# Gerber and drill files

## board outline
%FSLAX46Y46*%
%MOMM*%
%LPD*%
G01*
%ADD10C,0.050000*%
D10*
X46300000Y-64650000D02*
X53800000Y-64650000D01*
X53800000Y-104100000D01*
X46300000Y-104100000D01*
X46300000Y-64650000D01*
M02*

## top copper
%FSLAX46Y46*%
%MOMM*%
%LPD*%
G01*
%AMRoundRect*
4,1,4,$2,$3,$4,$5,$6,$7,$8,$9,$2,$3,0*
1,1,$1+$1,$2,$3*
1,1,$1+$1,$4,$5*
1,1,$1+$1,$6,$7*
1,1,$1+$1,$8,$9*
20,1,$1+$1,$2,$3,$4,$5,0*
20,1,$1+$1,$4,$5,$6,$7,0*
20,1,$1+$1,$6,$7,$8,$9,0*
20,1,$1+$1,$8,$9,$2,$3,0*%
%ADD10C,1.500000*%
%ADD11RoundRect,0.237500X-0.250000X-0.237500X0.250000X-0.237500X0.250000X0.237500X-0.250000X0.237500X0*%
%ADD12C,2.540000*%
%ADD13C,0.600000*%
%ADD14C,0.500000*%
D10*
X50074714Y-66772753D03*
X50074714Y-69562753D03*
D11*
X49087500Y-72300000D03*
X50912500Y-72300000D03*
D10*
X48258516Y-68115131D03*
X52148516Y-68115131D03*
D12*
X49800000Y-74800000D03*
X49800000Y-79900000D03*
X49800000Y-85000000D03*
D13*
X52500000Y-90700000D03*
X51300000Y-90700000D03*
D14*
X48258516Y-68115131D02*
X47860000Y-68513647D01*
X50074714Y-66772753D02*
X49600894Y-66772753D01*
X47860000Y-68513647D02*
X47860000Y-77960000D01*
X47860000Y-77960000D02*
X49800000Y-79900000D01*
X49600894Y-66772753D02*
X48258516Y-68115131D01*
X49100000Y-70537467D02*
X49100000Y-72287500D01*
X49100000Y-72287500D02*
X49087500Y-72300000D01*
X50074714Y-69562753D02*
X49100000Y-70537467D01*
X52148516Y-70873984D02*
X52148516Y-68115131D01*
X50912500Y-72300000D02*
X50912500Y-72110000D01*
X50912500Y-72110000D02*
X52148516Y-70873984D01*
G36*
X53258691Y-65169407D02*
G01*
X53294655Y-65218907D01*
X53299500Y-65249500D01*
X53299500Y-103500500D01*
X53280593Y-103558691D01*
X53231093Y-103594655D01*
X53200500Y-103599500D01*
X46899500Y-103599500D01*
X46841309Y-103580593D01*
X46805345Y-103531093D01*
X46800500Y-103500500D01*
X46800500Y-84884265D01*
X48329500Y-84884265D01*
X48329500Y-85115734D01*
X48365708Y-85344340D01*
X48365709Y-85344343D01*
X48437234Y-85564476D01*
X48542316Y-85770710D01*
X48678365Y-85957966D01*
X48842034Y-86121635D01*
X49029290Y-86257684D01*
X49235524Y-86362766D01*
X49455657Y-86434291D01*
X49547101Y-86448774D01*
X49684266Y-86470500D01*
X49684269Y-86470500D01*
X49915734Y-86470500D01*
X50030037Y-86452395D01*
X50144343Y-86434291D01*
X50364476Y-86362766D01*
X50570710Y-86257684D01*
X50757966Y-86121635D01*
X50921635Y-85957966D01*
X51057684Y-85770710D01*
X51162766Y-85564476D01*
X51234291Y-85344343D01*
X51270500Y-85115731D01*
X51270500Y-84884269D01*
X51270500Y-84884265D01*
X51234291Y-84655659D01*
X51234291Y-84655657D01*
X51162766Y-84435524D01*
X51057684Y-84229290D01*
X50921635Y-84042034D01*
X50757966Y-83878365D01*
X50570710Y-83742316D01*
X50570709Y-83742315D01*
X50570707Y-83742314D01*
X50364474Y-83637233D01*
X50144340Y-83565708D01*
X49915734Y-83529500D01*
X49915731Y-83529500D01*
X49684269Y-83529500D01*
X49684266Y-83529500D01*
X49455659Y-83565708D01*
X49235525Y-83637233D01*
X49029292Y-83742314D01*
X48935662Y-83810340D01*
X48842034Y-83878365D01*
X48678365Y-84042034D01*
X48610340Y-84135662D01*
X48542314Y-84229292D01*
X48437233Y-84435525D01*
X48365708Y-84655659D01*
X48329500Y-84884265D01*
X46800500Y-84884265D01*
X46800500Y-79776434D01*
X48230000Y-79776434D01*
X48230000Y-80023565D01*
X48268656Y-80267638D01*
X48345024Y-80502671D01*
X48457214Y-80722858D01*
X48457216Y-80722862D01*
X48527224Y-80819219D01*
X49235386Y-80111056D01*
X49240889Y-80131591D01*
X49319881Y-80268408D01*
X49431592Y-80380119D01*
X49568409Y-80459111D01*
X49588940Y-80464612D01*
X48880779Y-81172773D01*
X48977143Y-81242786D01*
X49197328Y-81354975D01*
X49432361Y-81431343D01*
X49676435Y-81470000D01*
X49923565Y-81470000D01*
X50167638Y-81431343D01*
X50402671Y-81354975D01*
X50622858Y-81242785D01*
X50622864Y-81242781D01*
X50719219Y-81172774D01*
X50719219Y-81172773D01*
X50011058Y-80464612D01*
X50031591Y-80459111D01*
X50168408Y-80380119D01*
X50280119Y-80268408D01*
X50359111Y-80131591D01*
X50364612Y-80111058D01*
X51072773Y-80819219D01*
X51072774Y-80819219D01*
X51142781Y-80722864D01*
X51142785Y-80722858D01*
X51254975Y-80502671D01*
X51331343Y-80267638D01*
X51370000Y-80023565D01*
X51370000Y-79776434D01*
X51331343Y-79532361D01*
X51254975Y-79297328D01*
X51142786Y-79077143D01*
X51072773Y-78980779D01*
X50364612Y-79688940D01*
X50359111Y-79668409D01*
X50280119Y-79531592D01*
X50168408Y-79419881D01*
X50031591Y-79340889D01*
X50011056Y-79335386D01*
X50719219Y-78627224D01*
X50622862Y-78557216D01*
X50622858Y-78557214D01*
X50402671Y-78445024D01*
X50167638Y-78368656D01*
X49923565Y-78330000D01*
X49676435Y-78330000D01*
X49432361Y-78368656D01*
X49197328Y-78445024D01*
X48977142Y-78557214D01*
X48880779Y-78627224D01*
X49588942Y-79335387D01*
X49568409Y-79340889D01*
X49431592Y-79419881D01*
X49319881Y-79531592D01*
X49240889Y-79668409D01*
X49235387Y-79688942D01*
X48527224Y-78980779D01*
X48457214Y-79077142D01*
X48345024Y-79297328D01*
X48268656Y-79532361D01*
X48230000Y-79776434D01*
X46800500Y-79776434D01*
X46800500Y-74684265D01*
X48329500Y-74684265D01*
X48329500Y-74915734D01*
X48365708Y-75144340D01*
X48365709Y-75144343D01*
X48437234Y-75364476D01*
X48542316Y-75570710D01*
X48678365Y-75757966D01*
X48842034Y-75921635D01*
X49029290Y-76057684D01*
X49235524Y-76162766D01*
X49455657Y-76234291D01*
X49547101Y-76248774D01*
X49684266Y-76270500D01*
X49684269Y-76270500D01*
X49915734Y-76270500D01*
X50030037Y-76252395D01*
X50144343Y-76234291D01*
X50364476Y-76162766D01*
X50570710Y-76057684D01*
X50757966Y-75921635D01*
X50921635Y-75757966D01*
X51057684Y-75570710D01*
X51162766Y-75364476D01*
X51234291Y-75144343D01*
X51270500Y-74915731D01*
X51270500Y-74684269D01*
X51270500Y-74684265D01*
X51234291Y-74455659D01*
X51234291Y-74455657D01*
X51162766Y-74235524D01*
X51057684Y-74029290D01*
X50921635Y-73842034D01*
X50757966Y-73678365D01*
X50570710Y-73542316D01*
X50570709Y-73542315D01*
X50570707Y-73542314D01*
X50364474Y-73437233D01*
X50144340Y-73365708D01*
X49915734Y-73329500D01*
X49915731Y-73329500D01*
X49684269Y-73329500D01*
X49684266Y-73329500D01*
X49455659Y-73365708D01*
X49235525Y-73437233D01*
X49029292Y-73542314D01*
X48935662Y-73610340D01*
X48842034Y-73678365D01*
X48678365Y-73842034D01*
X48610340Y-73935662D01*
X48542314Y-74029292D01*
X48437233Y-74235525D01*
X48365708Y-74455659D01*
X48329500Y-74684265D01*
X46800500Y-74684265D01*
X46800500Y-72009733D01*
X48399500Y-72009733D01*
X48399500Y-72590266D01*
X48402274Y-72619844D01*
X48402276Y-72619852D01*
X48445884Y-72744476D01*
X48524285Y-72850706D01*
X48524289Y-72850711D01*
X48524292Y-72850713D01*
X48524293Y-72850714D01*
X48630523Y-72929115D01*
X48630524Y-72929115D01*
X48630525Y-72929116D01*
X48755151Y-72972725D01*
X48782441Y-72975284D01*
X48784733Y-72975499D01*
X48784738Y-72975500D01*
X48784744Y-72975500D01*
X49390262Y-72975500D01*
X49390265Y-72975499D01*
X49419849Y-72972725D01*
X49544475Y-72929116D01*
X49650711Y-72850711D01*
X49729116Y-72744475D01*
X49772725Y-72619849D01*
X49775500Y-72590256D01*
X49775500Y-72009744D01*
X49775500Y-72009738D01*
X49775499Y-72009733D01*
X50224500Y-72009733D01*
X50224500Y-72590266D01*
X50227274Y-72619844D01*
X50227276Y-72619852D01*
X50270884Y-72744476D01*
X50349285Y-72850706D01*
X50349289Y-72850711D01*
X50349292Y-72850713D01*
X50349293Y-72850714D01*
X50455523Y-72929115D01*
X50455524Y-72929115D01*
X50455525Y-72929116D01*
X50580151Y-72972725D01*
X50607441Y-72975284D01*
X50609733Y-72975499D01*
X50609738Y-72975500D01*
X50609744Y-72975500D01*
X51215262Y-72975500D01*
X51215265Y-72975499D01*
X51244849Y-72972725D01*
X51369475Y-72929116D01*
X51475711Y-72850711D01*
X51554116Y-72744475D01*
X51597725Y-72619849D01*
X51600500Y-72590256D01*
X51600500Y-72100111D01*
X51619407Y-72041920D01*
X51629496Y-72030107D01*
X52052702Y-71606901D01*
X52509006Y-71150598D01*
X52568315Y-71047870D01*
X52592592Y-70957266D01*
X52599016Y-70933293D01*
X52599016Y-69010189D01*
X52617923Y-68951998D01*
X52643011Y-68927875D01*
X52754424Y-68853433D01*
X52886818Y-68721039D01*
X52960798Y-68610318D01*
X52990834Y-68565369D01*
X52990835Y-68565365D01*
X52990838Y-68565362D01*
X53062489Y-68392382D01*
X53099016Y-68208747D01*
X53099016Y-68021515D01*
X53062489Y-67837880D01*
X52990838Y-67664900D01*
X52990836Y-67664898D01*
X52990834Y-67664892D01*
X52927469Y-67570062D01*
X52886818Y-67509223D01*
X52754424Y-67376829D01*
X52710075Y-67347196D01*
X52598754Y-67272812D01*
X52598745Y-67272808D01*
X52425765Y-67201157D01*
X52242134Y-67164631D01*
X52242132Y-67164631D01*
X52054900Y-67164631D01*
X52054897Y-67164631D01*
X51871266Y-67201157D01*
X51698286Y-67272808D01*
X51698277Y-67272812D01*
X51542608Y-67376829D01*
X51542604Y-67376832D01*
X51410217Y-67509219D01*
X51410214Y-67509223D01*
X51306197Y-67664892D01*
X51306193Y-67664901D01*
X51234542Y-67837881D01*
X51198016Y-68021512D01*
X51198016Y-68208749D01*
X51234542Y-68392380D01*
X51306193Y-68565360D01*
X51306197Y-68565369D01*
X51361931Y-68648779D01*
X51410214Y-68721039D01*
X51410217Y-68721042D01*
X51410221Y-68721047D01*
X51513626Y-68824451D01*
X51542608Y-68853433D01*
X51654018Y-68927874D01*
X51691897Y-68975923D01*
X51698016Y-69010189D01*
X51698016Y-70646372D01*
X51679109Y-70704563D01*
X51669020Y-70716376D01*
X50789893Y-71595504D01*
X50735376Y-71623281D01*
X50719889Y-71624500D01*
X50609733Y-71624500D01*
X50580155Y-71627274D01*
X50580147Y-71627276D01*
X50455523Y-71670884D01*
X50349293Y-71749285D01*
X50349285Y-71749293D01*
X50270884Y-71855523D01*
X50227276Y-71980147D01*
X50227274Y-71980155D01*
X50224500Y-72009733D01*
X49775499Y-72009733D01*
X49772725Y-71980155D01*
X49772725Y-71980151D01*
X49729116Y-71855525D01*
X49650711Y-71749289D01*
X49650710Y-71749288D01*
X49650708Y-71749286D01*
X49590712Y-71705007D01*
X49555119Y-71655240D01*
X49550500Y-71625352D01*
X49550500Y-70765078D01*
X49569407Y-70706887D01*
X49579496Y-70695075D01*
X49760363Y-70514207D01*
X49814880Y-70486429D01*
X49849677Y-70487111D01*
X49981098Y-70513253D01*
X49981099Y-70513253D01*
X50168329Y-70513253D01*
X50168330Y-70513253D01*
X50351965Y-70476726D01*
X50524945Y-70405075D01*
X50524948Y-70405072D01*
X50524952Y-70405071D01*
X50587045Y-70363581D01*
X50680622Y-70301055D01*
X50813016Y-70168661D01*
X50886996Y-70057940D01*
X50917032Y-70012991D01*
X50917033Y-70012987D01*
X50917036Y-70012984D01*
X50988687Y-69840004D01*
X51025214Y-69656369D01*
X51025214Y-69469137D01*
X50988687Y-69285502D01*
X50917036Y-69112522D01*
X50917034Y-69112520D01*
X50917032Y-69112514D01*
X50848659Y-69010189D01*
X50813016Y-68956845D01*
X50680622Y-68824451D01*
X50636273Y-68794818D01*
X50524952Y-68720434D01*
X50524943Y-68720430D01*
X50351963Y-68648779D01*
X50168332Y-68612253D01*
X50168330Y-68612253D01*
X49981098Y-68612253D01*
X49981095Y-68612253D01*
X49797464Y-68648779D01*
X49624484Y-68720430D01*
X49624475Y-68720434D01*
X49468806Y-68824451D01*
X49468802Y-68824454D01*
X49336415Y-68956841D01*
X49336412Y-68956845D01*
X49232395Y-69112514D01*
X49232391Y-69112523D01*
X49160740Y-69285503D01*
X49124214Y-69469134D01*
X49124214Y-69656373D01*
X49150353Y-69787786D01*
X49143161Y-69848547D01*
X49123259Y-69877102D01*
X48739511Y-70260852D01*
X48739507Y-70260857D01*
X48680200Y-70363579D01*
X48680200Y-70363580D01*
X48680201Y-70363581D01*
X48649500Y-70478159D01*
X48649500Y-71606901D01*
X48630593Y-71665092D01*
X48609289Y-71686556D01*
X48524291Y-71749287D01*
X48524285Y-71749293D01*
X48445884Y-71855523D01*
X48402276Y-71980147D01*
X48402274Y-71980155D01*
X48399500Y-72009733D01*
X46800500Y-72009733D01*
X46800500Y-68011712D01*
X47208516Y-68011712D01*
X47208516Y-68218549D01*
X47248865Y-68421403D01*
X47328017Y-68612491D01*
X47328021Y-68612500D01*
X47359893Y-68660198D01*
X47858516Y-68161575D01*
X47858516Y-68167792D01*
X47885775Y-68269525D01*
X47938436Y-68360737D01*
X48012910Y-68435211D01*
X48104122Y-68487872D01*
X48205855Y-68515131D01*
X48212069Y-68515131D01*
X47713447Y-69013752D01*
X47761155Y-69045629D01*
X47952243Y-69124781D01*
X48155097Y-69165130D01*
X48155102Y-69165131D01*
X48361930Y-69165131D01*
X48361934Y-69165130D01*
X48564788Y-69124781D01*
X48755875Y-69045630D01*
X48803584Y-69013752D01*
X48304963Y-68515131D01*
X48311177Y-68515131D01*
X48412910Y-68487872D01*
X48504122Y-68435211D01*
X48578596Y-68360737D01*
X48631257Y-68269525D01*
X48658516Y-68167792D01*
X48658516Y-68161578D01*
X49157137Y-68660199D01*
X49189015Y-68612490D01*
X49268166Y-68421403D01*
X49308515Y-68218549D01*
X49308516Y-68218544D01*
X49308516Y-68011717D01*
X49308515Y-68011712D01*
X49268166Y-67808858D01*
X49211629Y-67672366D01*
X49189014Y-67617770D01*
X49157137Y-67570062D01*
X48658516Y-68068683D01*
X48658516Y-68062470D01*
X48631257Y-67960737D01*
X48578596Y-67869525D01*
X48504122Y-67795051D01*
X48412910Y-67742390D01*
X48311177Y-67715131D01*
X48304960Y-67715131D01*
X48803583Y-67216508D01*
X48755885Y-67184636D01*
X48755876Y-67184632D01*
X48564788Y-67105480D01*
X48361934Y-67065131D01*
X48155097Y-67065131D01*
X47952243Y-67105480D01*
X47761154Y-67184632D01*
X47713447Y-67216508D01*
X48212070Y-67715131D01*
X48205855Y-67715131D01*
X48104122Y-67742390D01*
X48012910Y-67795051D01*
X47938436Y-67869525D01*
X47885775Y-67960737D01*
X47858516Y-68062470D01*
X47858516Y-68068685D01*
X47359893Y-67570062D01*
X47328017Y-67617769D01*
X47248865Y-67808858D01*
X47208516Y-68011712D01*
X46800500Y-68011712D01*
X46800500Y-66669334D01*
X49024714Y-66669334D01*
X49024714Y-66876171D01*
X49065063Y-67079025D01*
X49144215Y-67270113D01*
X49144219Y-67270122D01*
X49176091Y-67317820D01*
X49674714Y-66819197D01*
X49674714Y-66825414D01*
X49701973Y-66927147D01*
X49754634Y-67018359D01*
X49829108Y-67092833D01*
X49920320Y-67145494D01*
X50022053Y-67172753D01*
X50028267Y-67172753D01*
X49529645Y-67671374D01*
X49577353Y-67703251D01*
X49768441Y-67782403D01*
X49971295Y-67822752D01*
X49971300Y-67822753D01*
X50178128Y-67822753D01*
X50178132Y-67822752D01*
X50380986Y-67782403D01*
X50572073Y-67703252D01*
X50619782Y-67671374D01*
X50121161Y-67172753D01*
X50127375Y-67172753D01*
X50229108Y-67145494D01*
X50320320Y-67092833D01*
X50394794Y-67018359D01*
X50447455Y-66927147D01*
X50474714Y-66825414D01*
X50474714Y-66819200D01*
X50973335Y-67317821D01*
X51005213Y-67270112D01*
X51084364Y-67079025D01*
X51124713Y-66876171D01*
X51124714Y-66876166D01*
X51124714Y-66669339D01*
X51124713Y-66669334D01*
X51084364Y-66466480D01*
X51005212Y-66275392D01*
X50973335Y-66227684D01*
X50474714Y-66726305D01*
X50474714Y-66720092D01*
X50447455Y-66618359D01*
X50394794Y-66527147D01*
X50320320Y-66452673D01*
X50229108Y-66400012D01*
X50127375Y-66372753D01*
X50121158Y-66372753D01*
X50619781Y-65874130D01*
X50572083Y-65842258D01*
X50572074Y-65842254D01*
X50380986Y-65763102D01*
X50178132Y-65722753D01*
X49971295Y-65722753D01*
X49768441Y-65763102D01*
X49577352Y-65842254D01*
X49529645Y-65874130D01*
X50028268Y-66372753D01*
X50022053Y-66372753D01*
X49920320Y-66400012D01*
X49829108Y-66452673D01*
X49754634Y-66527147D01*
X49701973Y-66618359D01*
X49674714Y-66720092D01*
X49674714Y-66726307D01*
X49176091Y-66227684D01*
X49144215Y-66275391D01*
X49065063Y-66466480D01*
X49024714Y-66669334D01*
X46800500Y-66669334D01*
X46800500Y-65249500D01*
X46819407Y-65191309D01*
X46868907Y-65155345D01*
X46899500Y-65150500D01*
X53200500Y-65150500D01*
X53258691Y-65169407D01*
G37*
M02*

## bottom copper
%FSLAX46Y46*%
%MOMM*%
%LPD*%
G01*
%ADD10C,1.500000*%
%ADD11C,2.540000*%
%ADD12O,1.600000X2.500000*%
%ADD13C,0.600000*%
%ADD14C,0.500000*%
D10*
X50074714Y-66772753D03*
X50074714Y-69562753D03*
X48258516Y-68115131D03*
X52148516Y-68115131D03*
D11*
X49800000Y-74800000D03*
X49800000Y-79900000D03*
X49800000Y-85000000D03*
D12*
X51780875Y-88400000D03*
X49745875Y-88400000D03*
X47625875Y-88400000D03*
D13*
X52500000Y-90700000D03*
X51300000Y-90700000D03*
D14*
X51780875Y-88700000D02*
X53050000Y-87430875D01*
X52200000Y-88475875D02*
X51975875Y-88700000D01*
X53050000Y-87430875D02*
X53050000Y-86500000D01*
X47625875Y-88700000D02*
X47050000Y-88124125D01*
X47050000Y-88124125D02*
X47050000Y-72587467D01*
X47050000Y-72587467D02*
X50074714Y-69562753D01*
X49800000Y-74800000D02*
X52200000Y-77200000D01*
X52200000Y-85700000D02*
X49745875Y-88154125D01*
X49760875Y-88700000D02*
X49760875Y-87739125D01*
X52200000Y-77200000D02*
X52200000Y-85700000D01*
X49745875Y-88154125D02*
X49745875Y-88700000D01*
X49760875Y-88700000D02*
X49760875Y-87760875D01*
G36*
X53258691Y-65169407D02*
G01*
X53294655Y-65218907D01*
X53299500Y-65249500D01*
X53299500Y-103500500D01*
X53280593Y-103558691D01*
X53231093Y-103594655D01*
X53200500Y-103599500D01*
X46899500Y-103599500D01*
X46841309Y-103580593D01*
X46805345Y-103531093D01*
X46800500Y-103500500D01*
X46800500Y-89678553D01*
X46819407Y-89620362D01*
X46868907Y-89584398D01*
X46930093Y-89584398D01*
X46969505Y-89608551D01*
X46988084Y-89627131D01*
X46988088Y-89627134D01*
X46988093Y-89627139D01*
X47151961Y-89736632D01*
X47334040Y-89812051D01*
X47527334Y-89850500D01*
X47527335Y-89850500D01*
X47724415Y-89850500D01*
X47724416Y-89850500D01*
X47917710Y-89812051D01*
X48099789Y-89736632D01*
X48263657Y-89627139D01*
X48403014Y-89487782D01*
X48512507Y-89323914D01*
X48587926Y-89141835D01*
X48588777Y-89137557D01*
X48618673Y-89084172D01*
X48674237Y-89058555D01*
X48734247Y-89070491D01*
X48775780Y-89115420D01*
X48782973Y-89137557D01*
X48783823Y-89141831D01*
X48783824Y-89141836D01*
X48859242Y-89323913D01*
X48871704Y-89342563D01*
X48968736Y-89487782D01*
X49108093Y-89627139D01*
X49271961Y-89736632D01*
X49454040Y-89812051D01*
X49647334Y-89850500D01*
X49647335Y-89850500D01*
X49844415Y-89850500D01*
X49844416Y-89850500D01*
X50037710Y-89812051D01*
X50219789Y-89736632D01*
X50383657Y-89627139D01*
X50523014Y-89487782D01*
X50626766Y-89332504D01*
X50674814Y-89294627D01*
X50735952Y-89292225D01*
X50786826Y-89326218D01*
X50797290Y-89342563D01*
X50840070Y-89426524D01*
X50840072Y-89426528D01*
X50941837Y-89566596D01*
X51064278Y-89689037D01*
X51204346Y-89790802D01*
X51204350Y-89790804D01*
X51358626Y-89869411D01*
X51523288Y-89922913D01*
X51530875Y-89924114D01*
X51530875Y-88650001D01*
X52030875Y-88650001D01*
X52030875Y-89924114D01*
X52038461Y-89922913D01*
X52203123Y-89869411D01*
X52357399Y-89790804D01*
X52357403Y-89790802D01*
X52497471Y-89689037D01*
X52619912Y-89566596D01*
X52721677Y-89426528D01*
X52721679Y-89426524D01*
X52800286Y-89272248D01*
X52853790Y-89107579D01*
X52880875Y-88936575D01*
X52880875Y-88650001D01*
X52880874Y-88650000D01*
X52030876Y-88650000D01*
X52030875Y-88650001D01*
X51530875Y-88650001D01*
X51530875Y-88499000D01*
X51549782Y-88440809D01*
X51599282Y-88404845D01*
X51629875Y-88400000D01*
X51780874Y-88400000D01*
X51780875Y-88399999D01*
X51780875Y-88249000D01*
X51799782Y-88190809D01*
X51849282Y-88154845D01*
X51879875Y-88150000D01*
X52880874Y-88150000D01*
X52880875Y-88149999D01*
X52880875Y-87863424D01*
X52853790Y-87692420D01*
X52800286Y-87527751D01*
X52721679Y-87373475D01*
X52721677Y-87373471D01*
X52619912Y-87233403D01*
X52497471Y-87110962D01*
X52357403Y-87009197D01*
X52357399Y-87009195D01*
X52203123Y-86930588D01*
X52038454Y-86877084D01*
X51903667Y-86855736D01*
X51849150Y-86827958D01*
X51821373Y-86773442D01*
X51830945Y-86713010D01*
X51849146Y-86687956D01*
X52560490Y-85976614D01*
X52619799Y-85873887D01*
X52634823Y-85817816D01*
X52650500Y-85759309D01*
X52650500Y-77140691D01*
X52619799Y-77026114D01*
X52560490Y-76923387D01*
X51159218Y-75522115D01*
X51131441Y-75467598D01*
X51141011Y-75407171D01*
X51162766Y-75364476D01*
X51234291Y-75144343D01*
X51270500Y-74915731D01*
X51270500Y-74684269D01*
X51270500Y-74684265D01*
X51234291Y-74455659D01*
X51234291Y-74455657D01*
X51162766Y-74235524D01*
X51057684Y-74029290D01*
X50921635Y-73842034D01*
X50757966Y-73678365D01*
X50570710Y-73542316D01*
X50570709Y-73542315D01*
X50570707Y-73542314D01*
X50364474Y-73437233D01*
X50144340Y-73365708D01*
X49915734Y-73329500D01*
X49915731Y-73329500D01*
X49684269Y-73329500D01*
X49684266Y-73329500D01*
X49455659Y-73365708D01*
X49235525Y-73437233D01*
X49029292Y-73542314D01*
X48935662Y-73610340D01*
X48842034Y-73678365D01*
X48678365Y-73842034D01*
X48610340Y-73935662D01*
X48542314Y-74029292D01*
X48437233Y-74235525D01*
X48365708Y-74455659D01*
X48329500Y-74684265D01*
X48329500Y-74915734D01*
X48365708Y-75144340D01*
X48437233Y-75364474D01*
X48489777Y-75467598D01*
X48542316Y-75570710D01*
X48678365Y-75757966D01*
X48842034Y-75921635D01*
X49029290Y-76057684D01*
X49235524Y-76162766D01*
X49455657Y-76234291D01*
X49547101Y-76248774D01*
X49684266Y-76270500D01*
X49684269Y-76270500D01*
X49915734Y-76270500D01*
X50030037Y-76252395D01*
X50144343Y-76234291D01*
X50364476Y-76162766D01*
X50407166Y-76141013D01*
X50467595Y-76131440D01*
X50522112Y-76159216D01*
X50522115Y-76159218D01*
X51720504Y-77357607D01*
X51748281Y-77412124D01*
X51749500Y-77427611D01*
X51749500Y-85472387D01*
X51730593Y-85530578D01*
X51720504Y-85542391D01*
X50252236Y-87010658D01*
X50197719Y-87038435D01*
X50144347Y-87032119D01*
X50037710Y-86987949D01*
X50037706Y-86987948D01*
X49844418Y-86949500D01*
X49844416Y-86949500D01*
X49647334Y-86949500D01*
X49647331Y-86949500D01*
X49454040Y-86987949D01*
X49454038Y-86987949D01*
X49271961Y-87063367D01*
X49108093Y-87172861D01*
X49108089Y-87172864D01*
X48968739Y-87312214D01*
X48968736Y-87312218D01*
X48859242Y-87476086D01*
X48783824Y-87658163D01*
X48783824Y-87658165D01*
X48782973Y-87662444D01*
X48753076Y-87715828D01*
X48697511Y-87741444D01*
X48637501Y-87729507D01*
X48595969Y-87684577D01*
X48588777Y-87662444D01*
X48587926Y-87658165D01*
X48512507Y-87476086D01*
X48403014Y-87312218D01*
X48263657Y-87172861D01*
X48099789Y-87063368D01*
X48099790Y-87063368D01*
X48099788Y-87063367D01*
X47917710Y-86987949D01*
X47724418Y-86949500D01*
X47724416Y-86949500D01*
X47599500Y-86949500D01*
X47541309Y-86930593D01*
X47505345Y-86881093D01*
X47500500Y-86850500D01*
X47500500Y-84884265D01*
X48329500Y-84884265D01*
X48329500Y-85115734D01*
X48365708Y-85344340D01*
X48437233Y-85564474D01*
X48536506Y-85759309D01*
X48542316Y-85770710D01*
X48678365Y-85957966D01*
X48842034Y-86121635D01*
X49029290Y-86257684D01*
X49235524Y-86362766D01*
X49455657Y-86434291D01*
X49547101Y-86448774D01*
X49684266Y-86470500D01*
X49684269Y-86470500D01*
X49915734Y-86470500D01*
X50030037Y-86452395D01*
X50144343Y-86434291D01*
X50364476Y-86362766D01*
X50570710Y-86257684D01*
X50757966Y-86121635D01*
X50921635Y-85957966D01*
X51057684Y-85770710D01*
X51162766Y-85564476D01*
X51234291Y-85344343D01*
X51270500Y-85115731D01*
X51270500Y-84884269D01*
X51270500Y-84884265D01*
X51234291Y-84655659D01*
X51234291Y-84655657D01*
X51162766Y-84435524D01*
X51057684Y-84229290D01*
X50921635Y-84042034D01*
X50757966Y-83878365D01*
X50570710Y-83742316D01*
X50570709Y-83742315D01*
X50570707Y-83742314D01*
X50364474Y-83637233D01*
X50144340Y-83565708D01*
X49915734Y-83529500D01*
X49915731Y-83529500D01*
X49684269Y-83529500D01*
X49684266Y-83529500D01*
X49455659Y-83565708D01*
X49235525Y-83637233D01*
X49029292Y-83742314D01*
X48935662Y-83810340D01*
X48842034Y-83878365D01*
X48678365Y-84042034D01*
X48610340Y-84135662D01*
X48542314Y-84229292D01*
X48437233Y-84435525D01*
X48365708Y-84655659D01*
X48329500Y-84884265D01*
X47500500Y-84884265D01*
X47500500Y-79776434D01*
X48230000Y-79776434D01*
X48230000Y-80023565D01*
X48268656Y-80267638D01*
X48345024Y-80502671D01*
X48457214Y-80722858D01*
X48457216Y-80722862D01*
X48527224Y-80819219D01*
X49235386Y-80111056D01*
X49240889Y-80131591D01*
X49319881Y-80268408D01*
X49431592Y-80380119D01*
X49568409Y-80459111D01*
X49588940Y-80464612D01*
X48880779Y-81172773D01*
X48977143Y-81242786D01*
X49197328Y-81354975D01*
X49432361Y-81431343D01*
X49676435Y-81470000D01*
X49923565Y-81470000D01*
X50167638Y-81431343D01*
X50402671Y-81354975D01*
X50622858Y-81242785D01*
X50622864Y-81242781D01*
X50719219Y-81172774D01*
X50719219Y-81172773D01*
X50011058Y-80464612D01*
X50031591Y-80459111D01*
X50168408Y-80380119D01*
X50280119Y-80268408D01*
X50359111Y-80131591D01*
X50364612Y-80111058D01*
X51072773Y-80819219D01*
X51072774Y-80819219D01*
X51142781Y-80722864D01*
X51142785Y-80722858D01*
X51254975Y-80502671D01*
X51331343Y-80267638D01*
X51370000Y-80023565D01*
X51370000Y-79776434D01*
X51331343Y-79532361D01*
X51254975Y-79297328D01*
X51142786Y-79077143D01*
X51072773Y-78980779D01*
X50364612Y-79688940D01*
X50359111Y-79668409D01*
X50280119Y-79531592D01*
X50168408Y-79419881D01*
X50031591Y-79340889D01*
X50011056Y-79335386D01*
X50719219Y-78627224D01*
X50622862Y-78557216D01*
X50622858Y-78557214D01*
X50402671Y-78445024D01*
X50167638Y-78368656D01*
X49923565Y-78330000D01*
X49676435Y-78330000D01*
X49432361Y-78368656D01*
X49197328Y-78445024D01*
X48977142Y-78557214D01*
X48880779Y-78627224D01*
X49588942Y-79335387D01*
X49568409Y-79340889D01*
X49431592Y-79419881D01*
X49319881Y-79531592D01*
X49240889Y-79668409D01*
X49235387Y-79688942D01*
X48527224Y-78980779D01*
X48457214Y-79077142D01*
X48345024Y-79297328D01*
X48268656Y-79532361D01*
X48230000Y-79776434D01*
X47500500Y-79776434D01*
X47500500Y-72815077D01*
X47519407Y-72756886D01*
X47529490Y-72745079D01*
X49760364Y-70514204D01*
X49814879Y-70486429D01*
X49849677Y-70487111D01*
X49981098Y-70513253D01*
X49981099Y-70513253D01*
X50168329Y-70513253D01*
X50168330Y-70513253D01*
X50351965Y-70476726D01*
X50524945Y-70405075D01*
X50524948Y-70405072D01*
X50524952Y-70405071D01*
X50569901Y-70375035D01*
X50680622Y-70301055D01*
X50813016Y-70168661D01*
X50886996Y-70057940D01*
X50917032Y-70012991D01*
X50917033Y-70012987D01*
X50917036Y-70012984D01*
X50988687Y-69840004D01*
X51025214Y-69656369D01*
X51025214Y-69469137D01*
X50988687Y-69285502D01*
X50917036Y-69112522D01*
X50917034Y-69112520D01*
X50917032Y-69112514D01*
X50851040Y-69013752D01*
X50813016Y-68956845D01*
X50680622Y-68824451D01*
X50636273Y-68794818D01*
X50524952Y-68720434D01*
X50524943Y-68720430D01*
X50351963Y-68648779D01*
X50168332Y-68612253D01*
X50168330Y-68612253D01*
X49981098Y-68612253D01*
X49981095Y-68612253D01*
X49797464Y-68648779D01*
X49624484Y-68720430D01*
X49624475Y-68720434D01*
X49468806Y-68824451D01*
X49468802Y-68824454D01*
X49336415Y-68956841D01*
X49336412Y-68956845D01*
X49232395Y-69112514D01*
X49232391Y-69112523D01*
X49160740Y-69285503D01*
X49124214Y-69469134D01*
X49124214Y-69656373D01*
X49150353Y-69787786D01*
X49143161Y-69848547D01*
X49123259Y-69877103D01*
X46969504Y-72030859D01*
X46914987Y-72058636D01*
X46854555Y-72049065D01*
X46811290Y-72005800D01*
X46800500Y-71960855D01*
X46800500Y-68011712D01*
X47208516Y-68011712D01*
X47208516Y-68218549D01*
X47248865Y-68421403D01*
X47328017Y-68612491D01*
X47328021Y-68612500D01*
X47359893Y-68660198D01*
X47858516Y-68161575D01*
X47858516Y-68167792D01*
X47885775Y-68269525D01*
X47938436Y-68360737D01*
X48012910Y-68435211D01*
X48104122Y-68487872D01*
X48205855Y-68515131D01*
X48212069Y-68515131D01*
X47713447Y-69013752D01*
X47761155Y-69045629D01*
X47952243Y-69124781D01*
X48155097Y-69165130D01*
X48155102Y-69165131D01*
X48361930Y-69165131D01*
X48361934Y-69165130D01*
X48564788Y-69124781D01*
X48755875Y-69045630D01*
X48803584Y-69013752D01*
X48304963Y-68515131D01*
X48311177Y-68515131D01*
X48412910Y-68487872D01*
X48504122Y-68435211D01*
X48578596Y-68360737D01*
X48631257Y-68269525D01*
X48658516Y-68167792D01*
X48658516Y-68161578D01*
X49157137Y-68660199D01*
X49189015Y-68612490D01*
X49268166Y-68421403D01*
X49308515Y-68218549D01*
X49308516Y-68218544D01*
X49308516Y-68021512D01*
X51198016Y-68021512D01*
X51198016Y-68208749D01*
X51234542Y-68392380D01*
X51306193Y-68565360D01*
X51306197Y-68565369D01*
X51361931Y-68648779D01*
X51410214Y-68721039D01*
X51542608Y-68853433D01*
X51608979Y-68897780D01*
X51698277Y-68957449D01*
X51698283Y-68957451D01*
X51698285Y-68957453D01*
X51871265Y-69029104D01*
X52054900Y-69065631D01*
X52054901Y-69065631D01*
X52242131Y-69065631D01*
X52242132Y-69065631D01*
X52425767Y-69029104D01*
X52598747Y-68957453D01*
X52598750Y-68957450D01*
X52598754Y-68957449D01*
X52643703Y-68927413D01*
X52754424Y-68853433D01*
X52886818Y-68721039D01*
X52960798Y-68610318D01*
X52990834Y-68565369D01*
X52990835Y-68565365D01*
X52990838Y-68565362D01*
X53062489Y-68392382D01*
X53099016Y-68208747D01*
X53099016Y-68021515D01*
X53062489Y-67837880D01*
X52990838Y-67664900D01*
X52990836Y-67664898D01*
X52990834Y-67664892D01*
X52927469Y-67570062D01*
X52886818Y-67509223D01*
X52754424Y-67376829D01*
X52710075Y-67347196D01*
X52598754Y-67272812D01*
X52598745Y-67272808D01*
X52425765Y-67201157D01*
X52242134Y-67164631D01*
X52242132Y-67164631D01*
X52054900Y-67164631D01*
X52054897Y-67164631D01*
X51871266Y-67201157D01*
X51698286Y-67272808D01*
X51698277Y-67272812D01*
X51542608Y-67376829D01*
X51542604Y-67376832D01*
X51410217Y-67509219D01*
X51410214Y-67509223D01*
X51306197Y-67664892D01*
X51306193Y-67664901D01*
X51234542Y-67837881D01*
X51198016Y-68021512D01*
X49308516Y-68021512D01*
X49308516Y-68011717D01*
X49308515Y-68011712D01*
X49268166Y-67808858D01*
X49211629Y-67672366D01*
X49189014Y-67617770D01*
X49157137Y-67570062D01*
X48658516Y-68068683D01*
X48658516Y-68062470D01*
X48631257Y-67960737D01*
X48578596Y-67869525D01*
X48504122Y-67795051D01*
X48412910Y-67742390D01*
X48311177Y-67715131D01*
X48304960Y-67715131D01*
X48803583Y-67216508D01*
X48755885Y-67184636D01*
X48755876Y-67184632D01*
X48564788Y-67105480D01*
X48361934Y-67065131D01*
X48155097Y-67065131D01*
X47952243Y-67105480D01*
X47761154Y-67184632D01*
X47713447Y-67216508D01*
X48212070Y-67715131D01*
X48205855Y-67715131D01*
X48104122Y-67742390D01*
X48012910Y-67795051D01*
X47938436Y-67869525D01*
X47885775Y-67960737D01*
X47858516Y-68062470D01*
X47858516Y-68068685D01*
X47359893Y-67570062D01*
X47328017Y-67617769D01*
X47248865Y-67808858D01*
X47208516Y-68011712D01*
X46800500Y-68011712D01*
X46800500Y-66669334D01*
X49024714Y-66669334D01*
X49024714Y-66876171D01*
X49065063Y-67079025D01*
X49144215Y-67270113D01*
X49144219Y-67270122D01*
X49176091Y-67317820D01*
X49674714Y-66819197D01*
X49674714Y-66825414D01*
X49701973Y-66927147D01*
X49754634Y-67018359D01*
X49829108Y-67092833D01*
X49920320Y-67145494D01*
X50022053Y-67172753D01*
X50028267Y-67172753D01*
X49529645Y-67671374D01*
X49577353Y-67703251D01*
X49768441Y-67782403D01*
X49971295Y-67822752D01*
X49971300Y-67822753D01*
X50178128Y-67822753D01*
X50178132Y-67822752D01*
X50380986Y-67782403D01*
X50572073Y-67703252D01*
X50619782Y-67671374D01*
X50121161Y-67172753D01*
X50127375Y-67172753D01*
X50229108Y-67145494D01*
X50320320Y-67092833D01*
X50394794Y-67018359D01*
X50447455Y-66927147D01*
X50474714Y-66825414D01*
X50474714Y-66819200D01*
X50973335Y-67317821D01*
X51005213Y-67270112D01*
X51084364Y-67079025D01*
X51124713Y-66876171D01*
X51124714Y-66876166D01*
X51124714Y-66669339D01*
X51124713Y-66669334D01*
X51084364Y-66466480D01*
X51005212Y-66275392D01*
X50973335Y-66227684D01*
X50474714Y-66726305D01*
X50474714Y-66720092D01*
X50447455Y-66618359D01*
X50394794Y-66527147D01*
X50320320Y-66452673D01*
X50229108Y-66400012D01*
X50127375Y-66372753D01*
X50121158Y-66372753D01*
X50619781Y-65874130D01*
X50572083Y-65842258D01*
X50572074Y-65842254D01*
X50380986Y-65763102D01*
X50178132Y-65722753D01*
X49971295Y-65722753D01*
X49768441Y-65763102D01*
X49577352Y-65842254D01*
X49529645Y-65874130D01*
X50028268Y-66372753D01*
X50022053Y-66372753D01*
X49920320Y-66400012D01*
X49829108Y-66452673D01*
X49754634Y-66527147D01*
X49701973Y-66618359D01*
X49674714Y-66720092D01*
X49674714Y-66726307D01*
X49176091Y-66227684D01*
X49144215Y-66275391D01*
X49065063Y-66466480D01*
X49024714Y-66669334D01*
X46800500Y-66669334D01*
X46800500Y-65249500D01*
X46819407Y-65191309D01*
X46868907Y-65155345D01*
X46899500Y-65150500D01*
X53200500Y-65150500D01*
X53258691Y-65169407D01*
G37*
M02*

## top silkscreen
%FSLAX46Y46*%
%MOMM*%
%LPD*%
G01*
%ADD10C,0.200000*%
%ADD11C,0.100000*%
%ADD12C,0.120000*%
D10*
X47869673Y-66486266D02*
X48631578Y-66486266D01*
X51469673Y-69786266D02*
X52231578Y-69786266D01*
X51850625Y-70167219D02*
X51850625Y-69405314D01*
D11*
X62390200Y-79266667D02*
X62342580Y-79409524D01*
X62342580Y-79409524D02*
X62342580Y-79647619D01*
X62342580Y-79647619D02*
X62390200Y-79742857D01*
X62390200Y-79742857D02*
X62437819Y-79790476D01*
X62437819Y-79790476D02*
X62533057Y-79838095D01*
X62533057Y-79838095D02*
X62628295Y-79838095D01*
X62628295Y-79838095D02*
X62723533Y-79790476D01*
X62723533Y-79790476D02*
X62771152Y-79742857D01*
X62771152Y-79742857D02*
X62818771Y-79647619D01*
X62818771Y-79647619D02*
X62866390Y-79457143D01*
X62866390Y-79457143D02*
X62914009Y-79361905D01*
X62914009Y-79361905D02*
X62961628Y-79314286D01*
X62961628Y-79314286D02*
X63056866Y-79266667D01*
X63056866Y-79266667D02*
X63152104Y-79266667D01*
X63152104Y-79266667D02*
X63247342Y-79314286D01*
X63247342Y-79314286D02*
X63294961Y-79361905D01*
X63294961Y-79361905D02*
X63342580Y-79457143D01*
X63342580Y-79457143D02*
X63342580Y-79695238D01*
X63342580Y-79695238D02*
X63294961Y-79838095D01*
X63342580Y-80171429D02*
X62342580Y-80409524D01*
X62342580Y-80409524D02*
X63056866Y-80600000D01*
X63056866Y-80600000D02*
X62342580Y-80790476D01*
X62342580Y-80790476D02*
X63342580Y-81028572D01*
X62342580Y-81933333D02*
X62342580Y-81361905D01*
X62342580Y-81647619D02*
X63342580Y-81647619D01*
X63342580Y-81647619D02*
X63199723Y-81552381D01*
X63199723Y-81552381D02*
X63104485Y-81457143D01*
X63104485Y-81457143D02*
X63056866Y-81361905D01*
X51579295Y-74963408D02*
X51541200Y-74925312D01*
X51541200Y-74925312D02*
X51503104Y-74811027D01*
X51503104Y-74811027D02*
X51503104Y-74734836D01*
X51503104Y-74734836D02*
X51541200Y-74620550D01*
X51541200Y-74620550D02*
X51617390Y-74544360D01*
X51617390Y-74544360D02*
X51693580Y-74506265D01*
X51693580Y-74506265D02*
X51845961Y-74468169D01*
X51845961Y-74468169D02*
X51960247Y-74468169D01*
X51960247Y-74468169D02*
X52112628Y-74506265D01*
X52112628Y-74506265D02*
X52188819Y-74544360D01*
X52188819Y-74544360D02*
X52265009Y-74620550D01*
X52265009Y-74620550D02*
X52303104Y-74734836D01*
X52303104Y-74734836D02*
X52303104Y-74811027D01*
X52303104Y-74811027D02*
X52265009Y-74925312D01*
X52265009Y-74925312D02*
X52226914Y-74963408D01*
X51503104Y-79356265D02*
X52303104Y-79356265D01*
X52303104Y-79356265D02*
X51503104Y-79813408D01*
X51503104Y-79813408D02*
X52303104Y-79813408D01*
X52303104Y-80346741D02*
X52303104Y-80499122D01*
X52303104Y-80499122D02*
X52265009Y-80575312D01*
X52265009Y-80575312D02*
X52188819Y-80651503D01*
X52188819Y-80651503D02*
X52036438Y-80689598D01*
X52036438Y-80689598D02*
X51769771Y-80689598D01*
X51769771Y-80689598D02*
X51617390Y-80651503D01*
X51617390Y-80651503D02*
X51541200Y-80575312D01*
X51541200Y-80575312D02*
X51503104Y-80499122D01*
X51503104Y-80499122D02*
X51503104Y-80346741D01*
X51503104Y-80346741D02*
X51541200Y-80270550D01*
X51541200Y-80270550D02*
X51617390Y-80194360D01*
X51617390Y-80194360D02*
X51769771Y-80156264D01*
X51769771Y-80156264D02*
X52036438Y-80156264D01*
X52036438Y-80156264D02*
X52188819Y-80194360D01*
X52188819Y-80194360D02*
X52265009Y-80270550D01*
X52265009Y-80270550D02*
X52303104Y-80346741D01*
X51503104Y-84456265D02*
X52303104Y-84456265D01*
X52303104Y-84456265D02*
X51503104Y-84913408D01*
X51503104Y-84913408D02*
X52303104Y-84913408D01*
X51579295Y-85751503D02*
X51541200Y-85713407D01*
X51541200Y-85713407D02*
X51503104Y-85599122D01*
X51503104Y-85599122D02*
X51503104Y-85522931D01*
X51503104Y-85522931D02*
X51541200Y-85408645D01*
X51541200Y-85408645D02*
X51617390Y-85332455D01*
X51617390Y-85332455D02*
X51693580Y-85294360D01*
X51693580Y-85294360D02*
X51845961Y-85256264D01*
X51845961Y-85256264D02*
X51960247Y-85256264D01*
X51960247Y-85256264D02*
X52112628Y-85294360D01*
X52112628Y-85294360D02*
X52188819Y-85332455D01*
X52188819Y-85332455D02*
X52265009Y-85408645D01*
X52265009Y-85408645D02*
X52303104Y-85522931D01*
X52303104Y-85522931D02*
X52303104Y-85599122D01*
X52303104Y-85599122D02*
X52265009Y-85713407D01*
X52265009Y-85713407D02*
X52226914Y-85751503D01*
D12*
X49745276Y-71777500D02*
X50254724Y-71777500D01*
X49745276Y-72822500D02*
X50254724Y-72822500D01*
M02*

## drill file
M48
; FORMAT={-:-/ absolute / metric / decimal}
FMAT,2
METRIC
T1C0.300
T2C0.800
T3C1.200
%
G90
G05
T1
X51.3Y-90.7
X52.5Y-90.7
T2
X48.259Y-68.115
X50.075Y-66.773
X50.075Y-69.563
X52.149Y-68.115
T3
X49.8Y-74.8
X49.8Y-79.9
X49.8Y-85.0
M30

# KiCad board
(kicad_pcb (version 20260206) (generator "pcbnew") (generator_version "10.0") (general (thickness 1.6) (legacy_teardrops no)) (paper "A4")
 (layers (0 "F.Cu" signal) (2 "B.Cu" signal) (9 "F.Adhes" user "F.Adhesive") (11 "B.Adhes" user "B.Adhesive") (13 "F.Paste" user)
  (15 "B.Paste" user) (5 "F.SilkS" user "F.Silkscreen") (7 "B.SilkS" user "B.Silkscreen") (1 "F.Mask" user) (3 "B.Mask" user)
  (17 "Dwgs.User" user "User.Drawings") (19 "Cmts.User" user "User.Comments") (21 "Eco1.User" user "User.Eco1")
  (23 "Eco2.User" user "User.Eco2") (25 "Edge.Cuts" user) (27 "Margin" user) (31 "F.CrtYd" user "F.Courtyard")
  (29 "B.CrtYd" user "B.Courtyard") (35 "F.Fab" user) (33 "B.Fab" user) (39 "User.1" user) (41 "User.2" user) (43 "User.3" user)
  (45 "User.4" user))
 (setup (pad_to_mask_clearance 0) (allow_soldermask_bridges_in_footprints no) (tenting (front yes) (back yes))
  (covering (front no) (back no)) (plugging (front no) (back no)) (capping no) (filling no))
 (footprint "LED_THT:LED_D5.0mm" (layer "F.Cu") (at 50.074714 66.872753 -90)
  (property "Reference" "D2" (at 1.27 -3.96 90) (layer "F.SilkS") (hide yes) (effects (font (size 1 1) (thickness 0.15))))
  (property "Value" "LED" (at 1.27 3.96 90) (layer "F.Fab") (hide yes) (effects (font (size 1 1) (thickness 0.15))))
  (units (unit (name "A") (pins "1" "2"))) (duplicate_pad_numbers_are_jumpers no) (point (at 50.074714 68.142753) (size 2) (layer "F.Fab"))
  (pad "1" thru_hole circle (at -0.1 0 270) (size 1.5 1.5) (drill 0.8) (layers "*.Cu" "*.Mask") (remove_unused_layers no) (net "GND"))
  (pad "2" thru_hole circle (at 2.69 0 270) (size 1.5 1.5) (drill 0.8) (layers "*.Cu" "*.Mask") (remove_unused_layers no) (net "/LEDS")))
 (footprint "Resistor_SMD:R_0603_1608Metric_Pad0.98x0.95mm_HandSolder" (layer "F.Cu") (at 50 72.3)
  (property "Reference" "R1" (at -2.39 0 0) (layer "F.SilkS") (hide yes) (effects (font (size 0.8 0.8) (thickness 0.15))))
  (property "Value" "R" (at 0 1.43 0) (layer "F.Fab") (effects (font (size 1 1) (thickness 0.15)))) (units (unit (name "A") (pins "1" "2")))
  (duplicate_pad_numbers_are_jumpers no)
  (fp_line (start -0.254724 -0.5225) (end 0.254724 -0.5225) (stroke (width 0.12) (type solid)) (layer "F.SilkS"))
  (fp_line (start -0.254724 0.5225) (end 0.254724 0.5225) (stroke (width 0.12) (type solid)) (layer "F.SilkS"))
  (pad "1" smd roundrect (at -0.9125 0) (size 0.975 0.95) (layers "F.Cu" "F.Mask" "F.Paste") (roundrect_rratio 0.25) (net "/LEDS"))
  (pad "2" smd roundrect (at 0.9125 0) (size 0.975 0.95) (layers "F.Cu" "F.Mask" "F.Paste") (roundrect_rratio 0.25) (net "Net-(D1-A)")))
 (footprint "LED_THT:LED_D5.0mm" (layer "F.Cu") (at 48.708516 68.115131)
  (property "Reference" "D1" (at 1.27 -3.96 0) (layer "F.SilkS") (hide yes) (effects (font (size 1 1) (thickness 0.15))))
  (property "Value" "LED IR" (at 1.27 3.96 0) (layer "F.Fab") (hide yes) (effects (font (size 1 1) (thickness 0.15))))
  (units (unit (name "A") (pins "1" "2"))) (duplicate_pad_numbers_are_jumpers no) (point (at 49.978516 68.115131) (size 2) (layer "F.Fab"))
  (pad "1" thru_hole circle (at -0.45 0) (size 1.5 1.5) (drill 0.8) (layers "*.Cu" "*.Mask") (remove_unused_layers no) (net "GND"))
  (pad "2" thru_hole circle (at 3.44 0) (size 1.5 1.5) (drill 0.8) (layers "*.Cu" "*.Mask") (remove_unused_layers no) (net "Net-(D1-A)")))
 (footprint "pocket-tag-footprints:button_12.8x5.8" (layer "F.Cu") (at 49.8 80.6 -90)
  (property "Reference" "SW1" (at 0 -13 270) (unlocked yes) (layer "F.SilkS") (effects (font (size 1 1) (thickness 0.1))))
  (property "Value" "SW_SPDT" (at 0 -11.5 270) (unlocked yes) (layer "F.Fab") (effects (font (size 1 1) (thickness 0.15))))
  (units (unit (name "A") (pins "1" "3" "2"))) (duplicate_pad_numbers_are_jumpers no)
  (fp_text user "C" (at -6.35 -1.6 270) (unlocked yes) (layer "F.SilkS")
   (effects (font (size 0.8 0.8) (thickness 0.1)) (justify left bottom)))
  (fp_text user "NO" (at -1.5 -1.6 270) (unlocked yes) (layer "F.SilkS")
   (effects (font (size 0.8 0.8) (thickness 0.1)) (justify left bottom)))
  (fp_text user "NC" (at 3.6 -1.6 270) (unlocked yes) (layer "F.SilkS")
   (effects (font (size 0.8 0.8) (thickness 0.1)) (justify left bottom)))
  (pad "1" thru_hole circle (at -5.8 0 270) (size 2.54 2.54) (drill 1.2) (layers "*.Cu" "*.Mask") (remove_unused_layers no) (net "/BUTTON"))
  (pad "2" thru_hole circle (at -0.7 0 270) (size 2.54 2.54) (drill 1.2) (layers "*.Cu" "*.Mask") (remove_unused_layers no) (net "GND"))
  (pad "3" thru_hole circle (at 4.4 0 270) (size 2.54 2.54) (drill 1.2) (layers "*.Cu" "*.Mask") (remove_unused_layers no)
   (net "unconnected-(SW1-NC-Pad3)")))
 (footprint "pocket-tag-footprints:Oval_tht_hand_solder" (layer "B.Cu") (at 51.780875 88.7 90)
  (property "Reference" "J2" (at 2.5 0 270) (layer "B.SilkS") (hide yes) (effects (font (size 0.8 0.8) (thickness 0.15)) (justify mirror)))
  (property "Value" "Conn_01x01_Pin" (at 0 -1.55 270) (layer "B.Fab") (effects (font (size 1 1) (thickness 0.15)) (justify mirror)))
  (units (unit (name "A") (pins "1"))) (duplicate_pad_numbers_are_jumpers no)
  (pad "1" smd oval (at 0 0 90) (size 2.5 1.6) (drill (offset 0.3 0)) (layers "B.Cu" "B.Mask" "B.Paste") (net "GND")))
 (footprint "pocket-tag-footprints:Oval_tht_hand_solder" (layer "B.Cu") (at 49.745875 88.7 90)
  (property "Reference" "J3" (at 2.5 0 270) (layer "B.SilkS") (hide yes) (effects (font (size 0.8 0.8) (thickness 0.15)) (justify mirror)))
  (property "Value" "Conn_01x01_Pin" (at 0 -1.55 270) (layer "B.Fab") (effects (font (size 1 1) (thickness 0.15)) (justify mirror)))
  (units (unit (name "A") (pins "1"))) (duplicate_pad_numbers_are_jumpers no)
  (pad "1" smd oval (at 0 0 90) (size 2.5 1.6) (drill (offset 0.3 0)) (layers "B.Cu" "B.Mask" "B.Paste") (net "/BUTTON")))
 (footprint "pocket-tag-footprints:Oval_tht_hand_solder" (layer "B.Cu") (at 47.625875 88.7 90)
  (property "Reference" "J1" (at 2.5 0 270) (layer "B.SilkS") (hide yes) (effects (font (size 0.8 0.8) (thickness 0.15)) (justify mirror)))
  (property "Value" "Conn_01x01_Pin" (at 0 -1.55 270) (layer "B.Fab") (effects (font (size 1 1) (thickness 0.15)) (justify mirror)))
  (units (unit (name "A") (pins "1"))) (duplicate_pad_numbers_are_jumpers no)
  (pad "1" smd oval (at 0 0 90) (size 2.5 1.6) (drill (offset 0.3 0)) (layers "B.Cu" "B.Mask" "B.Paste") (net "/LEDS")))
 (gr_rect (start 46.3 64.65) (end 53.8 104.1) (stroke (width 0.05) (type default)) (fill no) (layer "Edge.Cuts"))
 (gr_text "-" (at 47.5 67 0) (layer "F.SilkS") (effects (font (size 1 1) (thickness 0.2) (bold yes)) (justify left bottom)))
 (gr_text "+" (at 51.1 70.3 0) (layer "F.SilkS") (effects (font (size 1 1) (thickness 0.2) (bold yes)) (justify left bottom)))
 (segment (start 48.258516 68.115131) (end 47.86 68.513647) (width 0.5) (layer "F.Cu") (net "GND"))
 (segment (start 50.074714 66.772753) (end 49.600894 66.772753) (width 0.5) (layer "F.Cu") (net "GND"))
 (segment (start 47.86 68.513647) (end 47.86 77.96) (width 0.5) (layer "F.Cu") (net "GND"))
 (segment (start 47.86 77.96) (end 49.8 79.9) (width 0.5) (layer "F.Cu") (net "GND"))
 (segment (start 49.600894 66.772753) (end 48.258516 68.115131) (width 0.5) (layer "F.Cu") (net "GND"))
 (via (at 52.5 90.7) (size 0.6) (drill 0.3) (layers "F.Cu" "B.Cu") (free yes) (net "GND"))
 (via (at 51.3 90.7) (size 0.6) (drill 0.3) (layers "F.Cu" "B.Cu") (free yes) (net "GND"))
 (segment (start 51.780875 88.7) (end 53.05 87.430875) (width 0.5) (layer "B.Cu") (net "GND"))
 (segment (start 52.2 88.475875) (end 51.975875 88.7) (width 0.5) (layer "B.Cu") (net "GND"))
 (segment (start 53.05 87.430875) (end 53.05 86.5) (width 0.5) (layer "B.Cu") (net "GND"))
 (segment (start 49.1 70.537467) (end 49.1 72.2875) (width 0.5) (layer "F.Cu") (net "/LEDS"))
 (segment (start 49.1 72.2875) (end 49.0875 72.3) (width 0.5) (layer "F.Cu") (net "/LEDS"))
 (segment (start 50.074714 69.562753) (end 49.1 70.537467) (width 0.5) (layer "F.Cu") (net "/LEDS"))
 (segment (start 47.625875 88.7) (end 47.05 88.124125) (width 0.5) (layer "B.Cu") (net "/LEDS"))
 (segment (start 47.05 88.124125) (end 47.05 72.587467) (width 0.5) (layer "B.Cu") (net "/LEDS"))
 (segment (start 47.05 72.587467) (end 50.074714 69.562753) (width 0.5) (layer "B.Cu") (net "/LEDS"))
 (segment (start 52.148516 70.873984) (end 52.148516 68.115131) (width 0.5) (layer "F.Cu") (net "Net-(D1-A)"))
 (segment (start 50.9125 72.3) (end 50.9125 72.11) (width 0.5) (layer "F.Cu") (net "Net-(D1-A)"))
 (segment (start 50.9125 72.11) (end 52.148516 70.873984) (width 0.5) (layer "F.Cu") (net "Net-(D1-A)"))
 (segment (start 49.8 74.8) (end 52.2 77.2) (width 0.5) (layer "B.Cu") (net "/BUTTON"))
 (segment (start 52.2 85.7) (end 49.745875 88.154125) (width 0.5) (layer "B.Cu") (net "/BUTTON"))
 (segment (start 49.760875 88.7) (end 49.760875 87.739125) (width 0.5) (layer "B.Cu") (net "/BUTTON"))
 (segment (start 52.2 77.2) (end 52.2 85.7) (width 0.5) (layer "B.Cu") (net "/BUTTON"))
 (segment (start 49.745875 88.154125) (end 49.745875 88.7) (width 0.5) (layer "B.Cu") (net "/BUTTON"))
 (segment (start 49.760875 88.7) (end 49.760875 87.760875) (width 0.5) (layer "B.Cu") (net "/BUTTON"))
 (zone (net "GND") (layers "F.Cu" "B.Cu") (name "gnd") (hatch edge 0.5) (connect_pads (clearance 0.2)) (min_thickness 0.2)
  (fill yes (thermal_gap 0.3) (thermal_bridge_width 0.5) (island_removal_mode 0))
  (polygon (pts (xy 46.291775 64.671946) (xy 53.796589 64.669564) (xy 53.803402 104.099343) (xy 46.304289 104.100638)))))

